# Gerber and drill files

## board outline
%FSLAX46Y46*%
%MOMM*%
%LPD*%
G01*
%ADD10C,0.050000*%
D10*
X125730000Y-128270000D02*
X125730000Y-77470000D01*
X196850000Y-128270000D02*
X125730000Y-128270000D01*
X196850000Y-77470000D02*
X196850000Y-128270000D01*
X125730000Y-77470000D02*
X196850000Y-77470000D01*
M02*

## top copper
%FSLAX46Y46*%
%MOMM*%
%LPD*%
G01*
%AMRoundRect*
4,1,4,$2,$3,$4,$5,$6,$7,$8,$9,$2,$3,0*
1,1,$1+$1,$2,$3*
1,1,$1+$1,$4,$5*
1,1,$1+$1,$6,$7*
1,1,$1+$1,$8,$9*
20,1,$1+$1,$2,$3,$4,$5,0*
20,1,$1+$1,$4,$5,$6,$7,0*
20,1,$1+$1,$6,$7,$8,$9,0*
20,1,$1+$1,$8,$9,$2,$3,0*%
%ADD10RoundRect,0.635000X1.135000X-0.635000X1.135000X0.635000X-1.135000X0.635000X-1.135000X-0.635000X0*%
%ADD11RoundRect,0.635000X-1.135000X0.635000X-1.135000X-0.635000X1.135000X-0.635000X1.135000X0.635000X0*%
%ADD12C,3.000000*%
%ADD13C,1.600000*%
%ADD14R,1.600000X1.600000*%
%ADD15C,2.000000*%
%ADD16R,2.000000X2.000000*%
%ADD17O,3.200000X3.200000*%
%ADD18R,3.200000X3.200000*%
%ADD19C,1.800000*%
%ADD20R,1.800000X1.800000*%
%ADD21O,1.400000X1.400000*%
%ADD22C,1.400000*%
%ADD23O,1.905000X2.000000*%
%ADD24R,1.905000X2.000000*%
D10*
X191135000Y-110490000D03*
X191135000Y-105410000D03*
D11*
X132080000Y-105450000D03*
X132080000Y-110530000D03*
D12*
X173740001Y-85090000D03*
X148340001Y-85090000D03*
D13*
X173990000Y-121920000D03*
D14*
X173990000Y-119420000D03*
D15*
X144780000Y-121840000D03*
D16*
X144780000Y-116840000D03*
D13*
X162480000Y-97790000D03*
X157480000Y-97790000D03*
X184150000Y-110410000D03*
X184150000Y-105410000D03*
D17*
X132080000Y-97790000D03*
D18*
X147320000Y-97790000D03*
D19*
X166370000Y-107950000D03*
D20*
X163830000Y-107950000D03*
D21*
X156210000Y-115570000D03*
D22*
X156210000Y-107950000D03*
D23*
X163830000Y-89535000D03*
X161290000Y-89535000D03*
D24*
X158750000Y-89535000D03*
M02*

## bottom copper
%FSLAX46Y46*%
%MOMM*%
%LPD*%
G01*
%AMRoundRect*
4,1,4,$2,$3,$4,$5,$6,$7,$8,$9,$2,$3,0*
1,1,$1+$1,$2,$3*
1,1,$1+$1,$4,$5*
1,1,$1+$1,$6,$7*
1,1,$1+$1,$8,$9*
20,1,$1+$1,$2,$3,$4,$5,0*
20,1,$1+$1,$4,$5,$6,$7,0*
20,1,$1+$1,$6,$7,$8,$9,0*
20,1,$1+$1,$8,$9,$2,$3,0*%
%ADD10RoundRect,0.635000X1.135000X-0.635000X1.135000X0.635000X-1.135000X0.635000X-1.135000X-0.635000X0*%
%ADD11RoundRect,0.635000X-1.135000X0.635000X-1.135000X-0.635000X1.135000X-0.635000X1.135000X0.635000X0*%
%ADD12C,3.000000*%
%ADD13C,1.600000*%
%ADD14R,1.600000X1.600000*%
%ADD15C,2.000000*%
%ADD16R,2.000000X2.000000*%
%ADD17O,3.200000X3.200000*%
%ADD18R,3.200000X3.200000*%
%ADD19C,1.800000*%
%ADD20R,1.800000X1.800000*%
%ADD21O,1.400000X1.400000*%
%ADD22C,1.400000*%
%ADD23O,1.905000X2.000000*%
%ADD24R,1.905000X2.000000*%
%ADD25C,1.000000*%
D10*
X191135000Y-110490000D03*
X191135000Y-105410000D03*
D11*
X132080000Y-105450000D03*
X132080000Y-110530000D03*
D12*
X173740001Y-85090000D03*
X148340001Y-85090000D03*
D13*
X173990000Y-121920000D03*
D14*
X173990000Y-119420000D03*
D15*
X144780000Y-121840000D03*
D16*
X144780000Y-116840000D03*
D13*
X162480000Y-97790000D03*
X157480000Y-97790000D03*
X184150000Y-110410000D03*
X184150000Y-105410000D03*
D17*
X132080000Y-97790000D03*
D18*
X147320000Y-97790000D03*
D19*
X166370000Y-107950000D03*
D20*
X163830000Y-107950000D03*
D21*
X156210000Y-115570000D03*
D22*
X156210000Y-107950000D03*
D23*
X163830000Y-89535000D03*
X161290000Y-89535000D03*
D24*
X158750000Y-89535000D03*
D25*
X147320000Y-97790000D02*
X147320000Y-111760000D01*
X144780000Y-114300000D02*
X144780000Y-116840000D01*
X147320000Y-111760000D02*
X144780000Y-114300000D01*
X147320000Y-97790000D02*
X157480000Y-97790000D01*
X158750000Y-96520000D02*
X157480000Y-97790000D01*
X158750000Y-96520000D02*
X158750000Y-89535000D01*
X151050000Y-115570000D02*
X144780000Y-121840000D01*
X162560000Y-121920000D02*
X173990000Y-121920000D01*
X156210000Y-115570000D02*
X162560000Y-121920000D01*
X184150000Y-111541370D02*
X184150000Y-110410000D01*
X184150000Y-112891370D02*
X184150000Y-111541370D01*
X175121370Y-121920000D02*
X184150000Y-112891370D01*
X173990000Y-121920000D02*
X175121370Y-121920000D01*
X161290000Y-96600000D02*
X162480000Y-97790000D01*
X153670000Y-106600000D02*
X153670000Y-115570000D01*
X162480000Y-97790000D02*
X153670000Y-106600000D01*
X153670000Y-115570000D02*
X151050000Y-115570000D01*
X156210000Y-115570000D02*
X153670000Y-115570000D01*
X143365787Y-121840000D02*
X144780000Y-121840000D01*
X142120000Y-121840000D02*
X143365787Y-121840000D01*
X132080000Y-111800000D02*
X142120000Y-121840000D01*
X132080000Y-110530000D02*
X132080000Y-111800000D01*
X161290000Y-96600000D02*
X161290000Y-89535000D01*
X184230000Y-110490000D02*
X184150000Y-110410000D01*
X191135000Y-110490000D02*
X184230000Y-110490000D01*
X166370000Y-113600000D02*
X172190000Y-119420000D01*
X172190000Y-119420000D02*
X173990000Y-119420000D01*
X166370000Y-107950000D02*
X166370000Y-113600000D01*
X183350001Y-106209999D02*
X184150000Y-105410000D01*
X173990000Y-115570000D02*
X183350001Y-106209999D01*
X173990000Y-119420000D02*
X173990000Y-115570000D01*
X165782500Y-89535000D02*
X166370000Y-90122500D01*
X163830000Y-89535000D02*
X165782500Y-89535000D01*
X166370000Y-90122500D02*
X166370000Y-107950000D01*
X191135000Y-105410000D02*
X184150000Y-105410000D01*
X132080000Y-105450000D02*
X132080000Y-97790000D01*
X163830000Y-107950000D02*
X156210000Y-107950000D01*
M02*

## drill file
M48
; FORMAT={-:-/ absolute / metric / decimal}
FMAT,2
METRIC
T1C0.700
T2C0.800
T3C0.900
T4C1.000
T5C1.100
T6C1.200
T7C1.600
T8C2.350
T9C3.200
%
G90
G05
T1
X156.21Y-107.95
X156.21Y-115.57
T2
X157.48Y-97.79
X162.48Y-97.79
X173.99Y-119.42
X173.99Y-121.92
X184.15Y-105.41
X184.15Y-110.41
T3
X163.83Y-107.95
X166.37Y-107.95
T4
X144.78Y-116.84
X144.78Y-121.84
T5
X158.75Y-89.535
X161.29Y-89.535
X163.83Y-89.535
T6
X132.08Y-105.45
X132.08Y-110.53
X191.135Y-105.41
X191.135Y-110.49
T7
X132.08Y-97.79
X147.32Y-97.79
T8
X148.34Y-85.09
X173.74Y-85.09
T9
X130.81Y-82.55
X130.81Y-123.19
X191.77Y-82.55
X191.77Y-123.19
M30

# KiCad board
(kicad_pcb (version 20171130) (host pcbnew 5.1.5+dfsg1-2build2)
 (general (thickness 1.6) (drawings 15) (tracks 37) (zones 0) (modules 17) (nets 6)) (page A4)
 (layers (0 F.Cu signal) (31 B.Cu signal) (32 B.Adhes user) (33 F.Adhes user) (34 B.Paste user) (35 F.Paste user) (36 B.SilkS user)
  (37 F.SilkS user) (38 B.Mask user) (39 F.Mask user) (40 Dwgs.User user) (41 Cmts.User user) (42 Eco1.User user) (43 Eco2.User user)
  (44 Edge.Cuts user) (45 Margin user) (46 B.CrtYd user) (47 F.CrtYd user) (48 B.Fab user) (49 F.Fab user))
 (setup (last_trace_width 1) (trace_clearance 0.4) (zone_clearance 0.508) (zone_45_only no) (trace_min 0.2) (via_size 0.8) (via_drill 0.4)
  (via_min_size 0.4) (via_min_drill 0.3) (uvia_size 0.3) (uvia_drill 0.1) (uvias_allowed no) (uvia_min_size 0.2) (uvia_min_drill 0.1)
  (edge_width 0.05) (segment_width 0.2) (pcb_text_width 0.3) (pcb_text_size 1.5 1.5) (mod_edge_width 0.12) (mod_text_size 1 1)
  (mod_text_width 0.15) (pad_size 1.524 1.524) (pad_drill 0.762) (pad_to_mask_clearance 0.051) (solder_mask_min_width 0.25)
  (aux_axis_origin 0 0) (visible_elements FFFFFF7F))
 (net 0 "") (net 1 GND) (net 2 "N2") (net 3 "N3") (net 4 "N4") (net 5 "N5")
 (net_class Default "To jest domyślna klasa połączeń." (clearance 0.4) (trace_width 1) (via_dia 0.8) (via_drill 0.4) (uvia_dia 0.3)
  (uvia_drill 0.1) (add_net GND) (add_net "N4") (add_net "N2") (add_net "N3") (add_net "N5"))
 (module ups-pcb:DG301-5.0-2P (layer F.Cu) (at 191.135 107.99 90)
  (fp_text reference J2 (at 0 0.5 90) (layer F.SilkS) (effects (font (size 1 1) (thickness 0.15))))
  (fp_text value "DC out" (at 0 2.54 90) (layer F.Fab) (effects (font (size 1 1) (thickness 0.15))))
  (pad 1 thru_hole roundrect (at -2.5 0 90) (size 2.54 3.54) (drill 1.2) (layers *.Cu *.Mask) (roundrect_rratio 0.25) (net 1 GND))
  (pad 2 thru_hole roundrect (at 2.58 0 90) (size 2.54 3.54) (drill 1.2) (layers *.Cu *.Mask) (roundrect_rratio 0.25) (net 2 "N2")))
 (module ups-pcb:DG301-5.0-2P (layer F.Cu) (at 132.08 107.95 270)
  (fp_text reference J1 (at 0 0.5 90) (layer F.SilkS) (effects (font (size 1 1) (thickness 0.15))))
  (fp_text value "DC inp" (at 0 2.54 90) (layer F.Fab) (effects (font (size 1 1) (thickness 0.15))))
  (pad 1 thru_hole roundrect (at -2.5 0 270) (size 2.54 3.54) (drill 1.2) (layers *.Cu *.Mask) (roundrect_rratio 0.25) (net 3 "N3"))
  (pad 2 thru_hole roundrect (at 2.58 0 270) (size 2.54 3.54) (drill 1.2) (layers *.Cu *.Mask) (roundrect_rratio 0.25) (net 1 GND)))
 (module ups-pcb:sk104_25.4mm (layer F.Cu) (at 161.040001 85.09)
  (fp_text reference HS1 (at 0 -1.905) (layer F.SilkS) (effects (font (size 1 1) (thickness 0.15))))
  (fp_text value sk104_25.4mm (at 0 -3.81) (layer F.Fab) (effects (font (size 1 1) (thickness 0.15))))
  (pad "" np_thru_hole circle (at 12.7 0) (size 3 3) (drill 2.35) (layers *.Cu *.Mask))
  (pad "" np_thru_hole circle (at -12.7 0) (size 3 3) (drill 2.35) (layers *.Cu *.Mask)))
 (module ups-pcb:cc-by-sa (layer F.Cu) (at 159.385 121.92)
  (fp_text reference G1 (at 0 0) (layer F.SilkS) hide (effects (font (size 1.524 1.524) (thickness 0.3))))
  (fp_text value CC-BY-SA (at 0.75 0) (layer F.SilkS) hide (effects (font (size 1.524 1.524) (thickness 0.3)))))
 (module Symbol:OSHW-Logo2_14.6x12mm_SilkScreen (layer F.Cu) (at 186.055 93.98)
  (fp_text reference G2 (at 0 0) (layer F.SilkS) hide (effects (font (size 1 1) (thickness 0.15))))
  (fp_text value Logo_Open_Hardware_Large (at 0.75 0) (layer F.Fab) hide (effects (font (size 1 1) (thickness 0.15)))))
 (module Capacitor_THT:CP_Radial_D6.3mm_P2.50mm (layer F.Cu) (at 173.99 119.42 270)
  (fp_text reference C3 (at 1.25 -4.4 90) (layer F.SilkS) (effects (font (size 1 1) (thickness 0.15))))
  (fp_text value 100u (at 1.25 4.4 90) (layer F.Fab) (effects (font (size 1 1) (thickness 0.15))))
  (pad 2 thru_hole circle (at 2.5 0 270) (size 1.6 1.6) (drill 0.8) (layers *.Cu *.Mask) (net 1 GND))
  (pad 1 thru_hole rect (at 0 0 270) (size 1.6 1.6) (drill 0.8) (layers *.Cu *.Mask) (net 2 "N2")))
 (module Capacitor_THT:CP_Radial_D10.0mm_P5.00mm (layer F.Cu) (at 144.78 116.84 270)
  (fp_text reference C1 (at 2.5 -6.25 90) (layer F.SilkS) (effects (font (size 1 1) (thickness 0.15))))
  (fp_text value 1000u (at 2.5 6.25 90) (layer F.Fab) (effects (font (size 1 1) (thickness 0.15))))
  (pad 2 thru_hole circle (at 5 0 270) (size 2 2) (drill 1) (layers *.Cu *.Mask) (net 1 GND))
  (pad 1 thru_hole rect (at 0 0 270) (size 2 2) (drill 1) (layers *.Cu *.Mask) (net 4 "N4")))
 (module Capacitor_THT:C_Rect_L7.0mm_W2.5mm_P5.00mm (layer F.Cu) (at 157.48 97.79)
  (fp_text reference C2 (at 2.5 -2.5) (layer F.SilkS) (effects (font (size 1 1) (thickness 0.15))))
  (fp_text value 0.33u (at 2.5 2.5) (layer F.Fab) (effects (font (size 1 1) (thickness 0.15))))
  (pad 2 thru_hole circle (at 5 0) (size 1.6 1.6) (drill 0.8) (layers *.Cu *.Mask) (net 1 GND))
  (pad 1 thru_hole circle (at 0 0) (size 1.6 1.6) (drill 0.8) (layers *.Cu *.Mask) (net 4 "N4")))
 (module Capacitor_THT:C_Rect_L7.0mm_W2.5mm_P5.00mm (layer F.Cu) (at 184.15 105.41 270)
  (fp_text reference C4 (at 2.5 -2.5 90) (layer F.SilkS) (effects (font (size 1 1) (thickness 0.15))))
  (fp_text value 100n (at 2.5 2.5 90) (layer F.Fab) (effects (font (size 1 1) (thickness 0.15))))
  (pad 2 thru_hole circle (at 5 0 270) (size 1.6 1.6) (drill 0.8) (layers *.Cu *.Mask) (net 1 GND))
  (pad 1 thru_hole circle (at 0 0 270) (size 1.6 1.6) (drill 0.8) (layers *.Cu *.Mask) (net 2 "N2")))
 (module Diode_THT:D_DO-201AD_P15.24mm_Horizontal (layer F.Cu) (at 147.32 97.79 180)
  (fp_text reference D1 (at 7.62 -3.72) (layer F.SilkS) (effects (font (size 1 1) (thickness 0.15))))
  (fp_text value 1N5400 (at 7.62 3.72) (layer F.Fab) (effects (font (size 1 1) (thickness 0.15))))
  (pad 2 thru_hole oval (at 15.24 0 180) (size 3.2 3.2) (drill 1.6) (layers *.Cu *.Mask) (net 3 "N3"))
  (pad 1 thru_hole rect (at 0 0 180) (size 3.2 3.2) (drill 1.6) (layers *.Cu *.Mask) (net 4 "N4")))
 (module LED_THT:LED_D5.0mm (layer F.Cu) (at 163.83 107.95)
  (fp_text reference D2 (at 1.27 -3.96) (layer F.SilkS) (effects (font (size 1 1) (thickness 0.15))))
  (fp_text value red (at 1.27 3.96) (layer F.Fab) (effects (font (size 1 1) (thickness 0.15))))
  (pad 2 thru_hole circle (at 2.54 0) (size 1.8 1.8) (drill 0.9) (layers *.Cu *.Mask) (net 2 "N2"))
  (pad 1 thru_hole rect (at 0 0) (size 1.8 1.8) (drill 0.9) (layers *.Cu *.Mask) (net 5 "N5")))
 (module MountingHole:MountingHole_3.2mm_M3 (layer F.Cu) (at 130.81 82.55)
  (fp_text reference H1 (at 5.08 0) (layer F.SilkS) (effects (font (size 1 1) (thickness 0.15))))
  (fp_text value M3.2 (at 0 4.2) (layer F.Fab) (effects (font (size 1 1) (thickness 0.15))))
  (pad 1 np_thru_hole circle (at 0 0) (size 3.2 3.2) (drill 3.2) (layers *.Cu *.Mask)))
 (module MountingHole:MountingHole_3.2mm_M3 (layer F.Cu) (at 191.77 82.55)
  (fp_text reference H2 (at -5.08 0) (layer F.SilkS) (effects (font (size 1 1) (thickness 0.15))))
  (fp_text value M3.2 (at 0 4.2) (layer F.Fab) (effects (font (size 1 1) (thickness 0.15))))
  (pad 1 np_thru_hole circle (at 0 0) (size 3.2 3.2) (drill 3.2) (layers *.Cu *.Mask)))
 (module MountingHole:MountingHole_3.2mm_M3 (layer F.Cu) (at 191.77 123.19)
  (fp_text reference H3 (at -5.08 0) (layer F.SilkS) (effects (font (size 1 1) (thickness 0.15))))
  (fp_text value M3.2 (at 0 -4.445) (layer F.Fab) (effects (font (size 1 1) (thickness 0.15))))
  (pad 1 np_thru_hole circle (at 0 0) (size 3.2 3.2) (drill 3.2) (layers *.Cu *.Mask)))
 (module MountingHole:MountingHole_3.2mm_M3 (layer F.Cu) (at 130.81 123.19)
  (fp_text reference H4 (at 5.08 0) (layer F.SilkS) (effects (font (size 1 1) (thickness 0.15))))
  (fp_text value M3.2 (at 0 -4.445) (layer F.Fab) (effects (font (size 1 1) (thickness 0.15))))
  (pad 1 np_thru_hole circle (at 0 0) (size 3.2 3.2) (drill 3.2) (layers *.Cu *.Mask)))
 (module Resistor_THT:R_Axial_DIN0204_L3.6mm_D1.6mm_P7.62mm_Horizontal (layer F.Cu) (at 156.21 107.95 270)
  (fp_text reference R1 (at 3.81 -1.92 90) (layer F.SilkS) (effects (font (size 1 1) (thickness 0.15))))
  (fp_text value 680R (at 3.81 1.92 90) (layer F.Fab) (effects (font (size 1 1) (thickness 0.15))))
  (pad 2 thru_hole oval (at 7.62 0 270) (size 1.4 1.4) (drill 0.7) (layers *.Cu *.Mask) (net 1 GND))
  (pad 1 thru_hole circle (at 0 0 270) (size 1.4 1.4) (drill 0.7) (layers *.Cu *.Mask) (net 5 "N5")))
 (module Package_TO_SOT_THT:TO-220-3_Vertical (layer F.Cu) (at 158.75 89.535)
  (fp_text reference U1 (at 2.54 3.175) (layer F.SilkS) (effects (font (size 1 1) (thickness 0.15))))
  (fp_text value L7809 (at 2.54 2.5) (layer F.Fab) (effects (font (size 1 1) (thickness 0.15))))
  (pad 3 thru_hole oval (at 5.08 0) (size 1.905 2) (drill 1.1) (layers *.Cu *.Mask) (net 2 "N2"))
  (pad 2 thru_hole oval (at 2.54 0) (size 1.905 2) (drill 1.1) (layers *.Cu *.Mask) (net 1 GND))
  (pad 1 thru_hole rect (at 0 0) (size 1.905 2) (drill 1.1) (layers *.Cu *.Mask) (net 4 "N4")))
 (gr_line (start 125.73 128.27) (end 125.73 77.47) (layer Edge.Cuts) (width 0.05))
 (gr_line (start 196.85 128.27) (end 125.73 128.27) (layer Edge.Cuts) (width 0.05))
 (gr_line (start 196.85 77.47) (end 196.85 128.27) (layer Edge.Cuts) (width 0.05))
 (gr_line (start 125.73 77.47) (end 196.85 77.47) (layer Edge.Cuts) (width 0.05))
 (segment (start 147.32 97.79) (end 147.32 111.76) (width 1) (layer B.Cu) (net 4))
 (segment (start 144.78 114.3) (end 144.78 116.84) (width 1) (layer B.Cu) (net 4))
 (segment (start 147.32 111.76) (end 144.78 114.3) (width 1) (layer B.Cu) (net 4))
 (segment (start 147.32 97.79) (end 157.48 97.79) (width 1) (layer B.Cu) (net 4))
 (segment (start 158.75 96.52) (end 157.48 97.79) (width 1) (layer B.Cu) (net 4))
 (segment (start 158.75 96.52) (end 158.75 89.535) (width 1) (layer B.Cu) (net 4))
 (segment (start 151.05 115.57) (end 144.78 121.84) (width 1) (layer B.Cu) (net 1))
 (segment (start 162.56 121.92) (end 173.99 121.92) (width 1) (layer B.Cu) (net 1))
 (segment (start 156.21 115.57) (end 162.56 121.92) (width 1) (layer B.Cu) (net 1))
 (segment (start 184.15 111.54137) (end 184.15 110.41) (width 1) (layer B.Cu) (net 1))
 (segment (start 184.15 112.89137) (end 184.15 111.54137) (width 1) (layer B.Cu) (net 1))
 (segment (start 175.12137 121.92) (end 184.15 112.89137) (width 1) (layer B.Cu) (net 1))
 (segment (start 173.99 121.92) (end 175.12137 121.92) (width 1) (layer B.Cu) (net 1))
 (segment (start 161.29 96.6) (end 162.48 97.79) (width 1) (layer B.Cu) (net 1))
 (segment (start 153.67 106.6) (end 153.67 115.57) (width 1) (layer B.Cu) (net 1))
 (segment (start 162.48 97.79) (end 153.67 106.6) (width 1) (layer B.Cu) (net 1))
 (segment (start 153.67 115.57) (end 151.05 115.57) (width 1) (layer B.Cu) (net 1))
 (segment (start 156.21 115.57) (end 153.67 115.57) (width 1) (layer B.Cu) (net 1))
 (segment (start 143.365787 121.84) (end 144.78 121.84) (width 1) (layer B.Cu) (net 1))
 (segment (start 142.12 121.84) (end 143.365787 121.84) (width 1) (layer B.Cu) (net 1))
 (segment (start 132.08 111.8) (end 142.12 121.84) (width 1) (layer B.Cu) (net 1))
 (segment (start 132.08 110.53) (end 132.08 111.8) (width 1) (layer B.Cu) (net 1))
 (segment (start 161.29 96.6) (end 161.29 89.535) (width 1) (layer B.Cu) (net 1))
 (segment (start 184.23 110.49) (end 184.15 110.41) (width 1) (layer B.Cu) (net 1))
 (segment (start 191.135 110.49) (end 184.23 110.49) (width 1) (layer B.Cu) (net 1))
 (segment (start 166.37 113.6) (end 172.19 119.42) (width 1) (layer B.Cu) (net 2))
 (segment (start 172.19 119.42) (end 173.99 119.42) (width 1) (layer B.Cu) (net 2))
 (segment (start 166.37 107.95) (end 166.37 113.6) (width 1) (layer B.Cu) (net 2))
 (segment (start 183.350001 106.209999) (end 184.15 105.41) (width 1) (layer B.Cu) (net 2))
 (segment (start 173.99 115.57) (end 183.350001 106.209999) (width 1) (layer B.Cu) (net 2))
 (segment (start 173.99 119.42) (end 173.99 115.57) (width 1) (layer B.Cu) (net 2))
 (segment (start 165.7825 89.535) (end 166.37 90.1225) (width 1) (layer B.Cu) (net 2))
 (segment (start 163.83 89.535) (end 165.7825 89.535) (width 1) (layer B.Cu) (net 2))
 (segment (start 166.37 90.1225) (end 166.37 107.95) (width 1) (layer B.Cu) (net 2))
 (segment (start 191.135 105.41) (end 184.15 105.41) (width 1) (layer B.Cu) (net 2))
 (segment (start 132.08 105.45) (end 132.08 97.79) (width 1) (layer B.Cu) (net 3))
 (segment (start 163.83 107.95) (end 156.21 107.95) (width 1) (layer B.Cu) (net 5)))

